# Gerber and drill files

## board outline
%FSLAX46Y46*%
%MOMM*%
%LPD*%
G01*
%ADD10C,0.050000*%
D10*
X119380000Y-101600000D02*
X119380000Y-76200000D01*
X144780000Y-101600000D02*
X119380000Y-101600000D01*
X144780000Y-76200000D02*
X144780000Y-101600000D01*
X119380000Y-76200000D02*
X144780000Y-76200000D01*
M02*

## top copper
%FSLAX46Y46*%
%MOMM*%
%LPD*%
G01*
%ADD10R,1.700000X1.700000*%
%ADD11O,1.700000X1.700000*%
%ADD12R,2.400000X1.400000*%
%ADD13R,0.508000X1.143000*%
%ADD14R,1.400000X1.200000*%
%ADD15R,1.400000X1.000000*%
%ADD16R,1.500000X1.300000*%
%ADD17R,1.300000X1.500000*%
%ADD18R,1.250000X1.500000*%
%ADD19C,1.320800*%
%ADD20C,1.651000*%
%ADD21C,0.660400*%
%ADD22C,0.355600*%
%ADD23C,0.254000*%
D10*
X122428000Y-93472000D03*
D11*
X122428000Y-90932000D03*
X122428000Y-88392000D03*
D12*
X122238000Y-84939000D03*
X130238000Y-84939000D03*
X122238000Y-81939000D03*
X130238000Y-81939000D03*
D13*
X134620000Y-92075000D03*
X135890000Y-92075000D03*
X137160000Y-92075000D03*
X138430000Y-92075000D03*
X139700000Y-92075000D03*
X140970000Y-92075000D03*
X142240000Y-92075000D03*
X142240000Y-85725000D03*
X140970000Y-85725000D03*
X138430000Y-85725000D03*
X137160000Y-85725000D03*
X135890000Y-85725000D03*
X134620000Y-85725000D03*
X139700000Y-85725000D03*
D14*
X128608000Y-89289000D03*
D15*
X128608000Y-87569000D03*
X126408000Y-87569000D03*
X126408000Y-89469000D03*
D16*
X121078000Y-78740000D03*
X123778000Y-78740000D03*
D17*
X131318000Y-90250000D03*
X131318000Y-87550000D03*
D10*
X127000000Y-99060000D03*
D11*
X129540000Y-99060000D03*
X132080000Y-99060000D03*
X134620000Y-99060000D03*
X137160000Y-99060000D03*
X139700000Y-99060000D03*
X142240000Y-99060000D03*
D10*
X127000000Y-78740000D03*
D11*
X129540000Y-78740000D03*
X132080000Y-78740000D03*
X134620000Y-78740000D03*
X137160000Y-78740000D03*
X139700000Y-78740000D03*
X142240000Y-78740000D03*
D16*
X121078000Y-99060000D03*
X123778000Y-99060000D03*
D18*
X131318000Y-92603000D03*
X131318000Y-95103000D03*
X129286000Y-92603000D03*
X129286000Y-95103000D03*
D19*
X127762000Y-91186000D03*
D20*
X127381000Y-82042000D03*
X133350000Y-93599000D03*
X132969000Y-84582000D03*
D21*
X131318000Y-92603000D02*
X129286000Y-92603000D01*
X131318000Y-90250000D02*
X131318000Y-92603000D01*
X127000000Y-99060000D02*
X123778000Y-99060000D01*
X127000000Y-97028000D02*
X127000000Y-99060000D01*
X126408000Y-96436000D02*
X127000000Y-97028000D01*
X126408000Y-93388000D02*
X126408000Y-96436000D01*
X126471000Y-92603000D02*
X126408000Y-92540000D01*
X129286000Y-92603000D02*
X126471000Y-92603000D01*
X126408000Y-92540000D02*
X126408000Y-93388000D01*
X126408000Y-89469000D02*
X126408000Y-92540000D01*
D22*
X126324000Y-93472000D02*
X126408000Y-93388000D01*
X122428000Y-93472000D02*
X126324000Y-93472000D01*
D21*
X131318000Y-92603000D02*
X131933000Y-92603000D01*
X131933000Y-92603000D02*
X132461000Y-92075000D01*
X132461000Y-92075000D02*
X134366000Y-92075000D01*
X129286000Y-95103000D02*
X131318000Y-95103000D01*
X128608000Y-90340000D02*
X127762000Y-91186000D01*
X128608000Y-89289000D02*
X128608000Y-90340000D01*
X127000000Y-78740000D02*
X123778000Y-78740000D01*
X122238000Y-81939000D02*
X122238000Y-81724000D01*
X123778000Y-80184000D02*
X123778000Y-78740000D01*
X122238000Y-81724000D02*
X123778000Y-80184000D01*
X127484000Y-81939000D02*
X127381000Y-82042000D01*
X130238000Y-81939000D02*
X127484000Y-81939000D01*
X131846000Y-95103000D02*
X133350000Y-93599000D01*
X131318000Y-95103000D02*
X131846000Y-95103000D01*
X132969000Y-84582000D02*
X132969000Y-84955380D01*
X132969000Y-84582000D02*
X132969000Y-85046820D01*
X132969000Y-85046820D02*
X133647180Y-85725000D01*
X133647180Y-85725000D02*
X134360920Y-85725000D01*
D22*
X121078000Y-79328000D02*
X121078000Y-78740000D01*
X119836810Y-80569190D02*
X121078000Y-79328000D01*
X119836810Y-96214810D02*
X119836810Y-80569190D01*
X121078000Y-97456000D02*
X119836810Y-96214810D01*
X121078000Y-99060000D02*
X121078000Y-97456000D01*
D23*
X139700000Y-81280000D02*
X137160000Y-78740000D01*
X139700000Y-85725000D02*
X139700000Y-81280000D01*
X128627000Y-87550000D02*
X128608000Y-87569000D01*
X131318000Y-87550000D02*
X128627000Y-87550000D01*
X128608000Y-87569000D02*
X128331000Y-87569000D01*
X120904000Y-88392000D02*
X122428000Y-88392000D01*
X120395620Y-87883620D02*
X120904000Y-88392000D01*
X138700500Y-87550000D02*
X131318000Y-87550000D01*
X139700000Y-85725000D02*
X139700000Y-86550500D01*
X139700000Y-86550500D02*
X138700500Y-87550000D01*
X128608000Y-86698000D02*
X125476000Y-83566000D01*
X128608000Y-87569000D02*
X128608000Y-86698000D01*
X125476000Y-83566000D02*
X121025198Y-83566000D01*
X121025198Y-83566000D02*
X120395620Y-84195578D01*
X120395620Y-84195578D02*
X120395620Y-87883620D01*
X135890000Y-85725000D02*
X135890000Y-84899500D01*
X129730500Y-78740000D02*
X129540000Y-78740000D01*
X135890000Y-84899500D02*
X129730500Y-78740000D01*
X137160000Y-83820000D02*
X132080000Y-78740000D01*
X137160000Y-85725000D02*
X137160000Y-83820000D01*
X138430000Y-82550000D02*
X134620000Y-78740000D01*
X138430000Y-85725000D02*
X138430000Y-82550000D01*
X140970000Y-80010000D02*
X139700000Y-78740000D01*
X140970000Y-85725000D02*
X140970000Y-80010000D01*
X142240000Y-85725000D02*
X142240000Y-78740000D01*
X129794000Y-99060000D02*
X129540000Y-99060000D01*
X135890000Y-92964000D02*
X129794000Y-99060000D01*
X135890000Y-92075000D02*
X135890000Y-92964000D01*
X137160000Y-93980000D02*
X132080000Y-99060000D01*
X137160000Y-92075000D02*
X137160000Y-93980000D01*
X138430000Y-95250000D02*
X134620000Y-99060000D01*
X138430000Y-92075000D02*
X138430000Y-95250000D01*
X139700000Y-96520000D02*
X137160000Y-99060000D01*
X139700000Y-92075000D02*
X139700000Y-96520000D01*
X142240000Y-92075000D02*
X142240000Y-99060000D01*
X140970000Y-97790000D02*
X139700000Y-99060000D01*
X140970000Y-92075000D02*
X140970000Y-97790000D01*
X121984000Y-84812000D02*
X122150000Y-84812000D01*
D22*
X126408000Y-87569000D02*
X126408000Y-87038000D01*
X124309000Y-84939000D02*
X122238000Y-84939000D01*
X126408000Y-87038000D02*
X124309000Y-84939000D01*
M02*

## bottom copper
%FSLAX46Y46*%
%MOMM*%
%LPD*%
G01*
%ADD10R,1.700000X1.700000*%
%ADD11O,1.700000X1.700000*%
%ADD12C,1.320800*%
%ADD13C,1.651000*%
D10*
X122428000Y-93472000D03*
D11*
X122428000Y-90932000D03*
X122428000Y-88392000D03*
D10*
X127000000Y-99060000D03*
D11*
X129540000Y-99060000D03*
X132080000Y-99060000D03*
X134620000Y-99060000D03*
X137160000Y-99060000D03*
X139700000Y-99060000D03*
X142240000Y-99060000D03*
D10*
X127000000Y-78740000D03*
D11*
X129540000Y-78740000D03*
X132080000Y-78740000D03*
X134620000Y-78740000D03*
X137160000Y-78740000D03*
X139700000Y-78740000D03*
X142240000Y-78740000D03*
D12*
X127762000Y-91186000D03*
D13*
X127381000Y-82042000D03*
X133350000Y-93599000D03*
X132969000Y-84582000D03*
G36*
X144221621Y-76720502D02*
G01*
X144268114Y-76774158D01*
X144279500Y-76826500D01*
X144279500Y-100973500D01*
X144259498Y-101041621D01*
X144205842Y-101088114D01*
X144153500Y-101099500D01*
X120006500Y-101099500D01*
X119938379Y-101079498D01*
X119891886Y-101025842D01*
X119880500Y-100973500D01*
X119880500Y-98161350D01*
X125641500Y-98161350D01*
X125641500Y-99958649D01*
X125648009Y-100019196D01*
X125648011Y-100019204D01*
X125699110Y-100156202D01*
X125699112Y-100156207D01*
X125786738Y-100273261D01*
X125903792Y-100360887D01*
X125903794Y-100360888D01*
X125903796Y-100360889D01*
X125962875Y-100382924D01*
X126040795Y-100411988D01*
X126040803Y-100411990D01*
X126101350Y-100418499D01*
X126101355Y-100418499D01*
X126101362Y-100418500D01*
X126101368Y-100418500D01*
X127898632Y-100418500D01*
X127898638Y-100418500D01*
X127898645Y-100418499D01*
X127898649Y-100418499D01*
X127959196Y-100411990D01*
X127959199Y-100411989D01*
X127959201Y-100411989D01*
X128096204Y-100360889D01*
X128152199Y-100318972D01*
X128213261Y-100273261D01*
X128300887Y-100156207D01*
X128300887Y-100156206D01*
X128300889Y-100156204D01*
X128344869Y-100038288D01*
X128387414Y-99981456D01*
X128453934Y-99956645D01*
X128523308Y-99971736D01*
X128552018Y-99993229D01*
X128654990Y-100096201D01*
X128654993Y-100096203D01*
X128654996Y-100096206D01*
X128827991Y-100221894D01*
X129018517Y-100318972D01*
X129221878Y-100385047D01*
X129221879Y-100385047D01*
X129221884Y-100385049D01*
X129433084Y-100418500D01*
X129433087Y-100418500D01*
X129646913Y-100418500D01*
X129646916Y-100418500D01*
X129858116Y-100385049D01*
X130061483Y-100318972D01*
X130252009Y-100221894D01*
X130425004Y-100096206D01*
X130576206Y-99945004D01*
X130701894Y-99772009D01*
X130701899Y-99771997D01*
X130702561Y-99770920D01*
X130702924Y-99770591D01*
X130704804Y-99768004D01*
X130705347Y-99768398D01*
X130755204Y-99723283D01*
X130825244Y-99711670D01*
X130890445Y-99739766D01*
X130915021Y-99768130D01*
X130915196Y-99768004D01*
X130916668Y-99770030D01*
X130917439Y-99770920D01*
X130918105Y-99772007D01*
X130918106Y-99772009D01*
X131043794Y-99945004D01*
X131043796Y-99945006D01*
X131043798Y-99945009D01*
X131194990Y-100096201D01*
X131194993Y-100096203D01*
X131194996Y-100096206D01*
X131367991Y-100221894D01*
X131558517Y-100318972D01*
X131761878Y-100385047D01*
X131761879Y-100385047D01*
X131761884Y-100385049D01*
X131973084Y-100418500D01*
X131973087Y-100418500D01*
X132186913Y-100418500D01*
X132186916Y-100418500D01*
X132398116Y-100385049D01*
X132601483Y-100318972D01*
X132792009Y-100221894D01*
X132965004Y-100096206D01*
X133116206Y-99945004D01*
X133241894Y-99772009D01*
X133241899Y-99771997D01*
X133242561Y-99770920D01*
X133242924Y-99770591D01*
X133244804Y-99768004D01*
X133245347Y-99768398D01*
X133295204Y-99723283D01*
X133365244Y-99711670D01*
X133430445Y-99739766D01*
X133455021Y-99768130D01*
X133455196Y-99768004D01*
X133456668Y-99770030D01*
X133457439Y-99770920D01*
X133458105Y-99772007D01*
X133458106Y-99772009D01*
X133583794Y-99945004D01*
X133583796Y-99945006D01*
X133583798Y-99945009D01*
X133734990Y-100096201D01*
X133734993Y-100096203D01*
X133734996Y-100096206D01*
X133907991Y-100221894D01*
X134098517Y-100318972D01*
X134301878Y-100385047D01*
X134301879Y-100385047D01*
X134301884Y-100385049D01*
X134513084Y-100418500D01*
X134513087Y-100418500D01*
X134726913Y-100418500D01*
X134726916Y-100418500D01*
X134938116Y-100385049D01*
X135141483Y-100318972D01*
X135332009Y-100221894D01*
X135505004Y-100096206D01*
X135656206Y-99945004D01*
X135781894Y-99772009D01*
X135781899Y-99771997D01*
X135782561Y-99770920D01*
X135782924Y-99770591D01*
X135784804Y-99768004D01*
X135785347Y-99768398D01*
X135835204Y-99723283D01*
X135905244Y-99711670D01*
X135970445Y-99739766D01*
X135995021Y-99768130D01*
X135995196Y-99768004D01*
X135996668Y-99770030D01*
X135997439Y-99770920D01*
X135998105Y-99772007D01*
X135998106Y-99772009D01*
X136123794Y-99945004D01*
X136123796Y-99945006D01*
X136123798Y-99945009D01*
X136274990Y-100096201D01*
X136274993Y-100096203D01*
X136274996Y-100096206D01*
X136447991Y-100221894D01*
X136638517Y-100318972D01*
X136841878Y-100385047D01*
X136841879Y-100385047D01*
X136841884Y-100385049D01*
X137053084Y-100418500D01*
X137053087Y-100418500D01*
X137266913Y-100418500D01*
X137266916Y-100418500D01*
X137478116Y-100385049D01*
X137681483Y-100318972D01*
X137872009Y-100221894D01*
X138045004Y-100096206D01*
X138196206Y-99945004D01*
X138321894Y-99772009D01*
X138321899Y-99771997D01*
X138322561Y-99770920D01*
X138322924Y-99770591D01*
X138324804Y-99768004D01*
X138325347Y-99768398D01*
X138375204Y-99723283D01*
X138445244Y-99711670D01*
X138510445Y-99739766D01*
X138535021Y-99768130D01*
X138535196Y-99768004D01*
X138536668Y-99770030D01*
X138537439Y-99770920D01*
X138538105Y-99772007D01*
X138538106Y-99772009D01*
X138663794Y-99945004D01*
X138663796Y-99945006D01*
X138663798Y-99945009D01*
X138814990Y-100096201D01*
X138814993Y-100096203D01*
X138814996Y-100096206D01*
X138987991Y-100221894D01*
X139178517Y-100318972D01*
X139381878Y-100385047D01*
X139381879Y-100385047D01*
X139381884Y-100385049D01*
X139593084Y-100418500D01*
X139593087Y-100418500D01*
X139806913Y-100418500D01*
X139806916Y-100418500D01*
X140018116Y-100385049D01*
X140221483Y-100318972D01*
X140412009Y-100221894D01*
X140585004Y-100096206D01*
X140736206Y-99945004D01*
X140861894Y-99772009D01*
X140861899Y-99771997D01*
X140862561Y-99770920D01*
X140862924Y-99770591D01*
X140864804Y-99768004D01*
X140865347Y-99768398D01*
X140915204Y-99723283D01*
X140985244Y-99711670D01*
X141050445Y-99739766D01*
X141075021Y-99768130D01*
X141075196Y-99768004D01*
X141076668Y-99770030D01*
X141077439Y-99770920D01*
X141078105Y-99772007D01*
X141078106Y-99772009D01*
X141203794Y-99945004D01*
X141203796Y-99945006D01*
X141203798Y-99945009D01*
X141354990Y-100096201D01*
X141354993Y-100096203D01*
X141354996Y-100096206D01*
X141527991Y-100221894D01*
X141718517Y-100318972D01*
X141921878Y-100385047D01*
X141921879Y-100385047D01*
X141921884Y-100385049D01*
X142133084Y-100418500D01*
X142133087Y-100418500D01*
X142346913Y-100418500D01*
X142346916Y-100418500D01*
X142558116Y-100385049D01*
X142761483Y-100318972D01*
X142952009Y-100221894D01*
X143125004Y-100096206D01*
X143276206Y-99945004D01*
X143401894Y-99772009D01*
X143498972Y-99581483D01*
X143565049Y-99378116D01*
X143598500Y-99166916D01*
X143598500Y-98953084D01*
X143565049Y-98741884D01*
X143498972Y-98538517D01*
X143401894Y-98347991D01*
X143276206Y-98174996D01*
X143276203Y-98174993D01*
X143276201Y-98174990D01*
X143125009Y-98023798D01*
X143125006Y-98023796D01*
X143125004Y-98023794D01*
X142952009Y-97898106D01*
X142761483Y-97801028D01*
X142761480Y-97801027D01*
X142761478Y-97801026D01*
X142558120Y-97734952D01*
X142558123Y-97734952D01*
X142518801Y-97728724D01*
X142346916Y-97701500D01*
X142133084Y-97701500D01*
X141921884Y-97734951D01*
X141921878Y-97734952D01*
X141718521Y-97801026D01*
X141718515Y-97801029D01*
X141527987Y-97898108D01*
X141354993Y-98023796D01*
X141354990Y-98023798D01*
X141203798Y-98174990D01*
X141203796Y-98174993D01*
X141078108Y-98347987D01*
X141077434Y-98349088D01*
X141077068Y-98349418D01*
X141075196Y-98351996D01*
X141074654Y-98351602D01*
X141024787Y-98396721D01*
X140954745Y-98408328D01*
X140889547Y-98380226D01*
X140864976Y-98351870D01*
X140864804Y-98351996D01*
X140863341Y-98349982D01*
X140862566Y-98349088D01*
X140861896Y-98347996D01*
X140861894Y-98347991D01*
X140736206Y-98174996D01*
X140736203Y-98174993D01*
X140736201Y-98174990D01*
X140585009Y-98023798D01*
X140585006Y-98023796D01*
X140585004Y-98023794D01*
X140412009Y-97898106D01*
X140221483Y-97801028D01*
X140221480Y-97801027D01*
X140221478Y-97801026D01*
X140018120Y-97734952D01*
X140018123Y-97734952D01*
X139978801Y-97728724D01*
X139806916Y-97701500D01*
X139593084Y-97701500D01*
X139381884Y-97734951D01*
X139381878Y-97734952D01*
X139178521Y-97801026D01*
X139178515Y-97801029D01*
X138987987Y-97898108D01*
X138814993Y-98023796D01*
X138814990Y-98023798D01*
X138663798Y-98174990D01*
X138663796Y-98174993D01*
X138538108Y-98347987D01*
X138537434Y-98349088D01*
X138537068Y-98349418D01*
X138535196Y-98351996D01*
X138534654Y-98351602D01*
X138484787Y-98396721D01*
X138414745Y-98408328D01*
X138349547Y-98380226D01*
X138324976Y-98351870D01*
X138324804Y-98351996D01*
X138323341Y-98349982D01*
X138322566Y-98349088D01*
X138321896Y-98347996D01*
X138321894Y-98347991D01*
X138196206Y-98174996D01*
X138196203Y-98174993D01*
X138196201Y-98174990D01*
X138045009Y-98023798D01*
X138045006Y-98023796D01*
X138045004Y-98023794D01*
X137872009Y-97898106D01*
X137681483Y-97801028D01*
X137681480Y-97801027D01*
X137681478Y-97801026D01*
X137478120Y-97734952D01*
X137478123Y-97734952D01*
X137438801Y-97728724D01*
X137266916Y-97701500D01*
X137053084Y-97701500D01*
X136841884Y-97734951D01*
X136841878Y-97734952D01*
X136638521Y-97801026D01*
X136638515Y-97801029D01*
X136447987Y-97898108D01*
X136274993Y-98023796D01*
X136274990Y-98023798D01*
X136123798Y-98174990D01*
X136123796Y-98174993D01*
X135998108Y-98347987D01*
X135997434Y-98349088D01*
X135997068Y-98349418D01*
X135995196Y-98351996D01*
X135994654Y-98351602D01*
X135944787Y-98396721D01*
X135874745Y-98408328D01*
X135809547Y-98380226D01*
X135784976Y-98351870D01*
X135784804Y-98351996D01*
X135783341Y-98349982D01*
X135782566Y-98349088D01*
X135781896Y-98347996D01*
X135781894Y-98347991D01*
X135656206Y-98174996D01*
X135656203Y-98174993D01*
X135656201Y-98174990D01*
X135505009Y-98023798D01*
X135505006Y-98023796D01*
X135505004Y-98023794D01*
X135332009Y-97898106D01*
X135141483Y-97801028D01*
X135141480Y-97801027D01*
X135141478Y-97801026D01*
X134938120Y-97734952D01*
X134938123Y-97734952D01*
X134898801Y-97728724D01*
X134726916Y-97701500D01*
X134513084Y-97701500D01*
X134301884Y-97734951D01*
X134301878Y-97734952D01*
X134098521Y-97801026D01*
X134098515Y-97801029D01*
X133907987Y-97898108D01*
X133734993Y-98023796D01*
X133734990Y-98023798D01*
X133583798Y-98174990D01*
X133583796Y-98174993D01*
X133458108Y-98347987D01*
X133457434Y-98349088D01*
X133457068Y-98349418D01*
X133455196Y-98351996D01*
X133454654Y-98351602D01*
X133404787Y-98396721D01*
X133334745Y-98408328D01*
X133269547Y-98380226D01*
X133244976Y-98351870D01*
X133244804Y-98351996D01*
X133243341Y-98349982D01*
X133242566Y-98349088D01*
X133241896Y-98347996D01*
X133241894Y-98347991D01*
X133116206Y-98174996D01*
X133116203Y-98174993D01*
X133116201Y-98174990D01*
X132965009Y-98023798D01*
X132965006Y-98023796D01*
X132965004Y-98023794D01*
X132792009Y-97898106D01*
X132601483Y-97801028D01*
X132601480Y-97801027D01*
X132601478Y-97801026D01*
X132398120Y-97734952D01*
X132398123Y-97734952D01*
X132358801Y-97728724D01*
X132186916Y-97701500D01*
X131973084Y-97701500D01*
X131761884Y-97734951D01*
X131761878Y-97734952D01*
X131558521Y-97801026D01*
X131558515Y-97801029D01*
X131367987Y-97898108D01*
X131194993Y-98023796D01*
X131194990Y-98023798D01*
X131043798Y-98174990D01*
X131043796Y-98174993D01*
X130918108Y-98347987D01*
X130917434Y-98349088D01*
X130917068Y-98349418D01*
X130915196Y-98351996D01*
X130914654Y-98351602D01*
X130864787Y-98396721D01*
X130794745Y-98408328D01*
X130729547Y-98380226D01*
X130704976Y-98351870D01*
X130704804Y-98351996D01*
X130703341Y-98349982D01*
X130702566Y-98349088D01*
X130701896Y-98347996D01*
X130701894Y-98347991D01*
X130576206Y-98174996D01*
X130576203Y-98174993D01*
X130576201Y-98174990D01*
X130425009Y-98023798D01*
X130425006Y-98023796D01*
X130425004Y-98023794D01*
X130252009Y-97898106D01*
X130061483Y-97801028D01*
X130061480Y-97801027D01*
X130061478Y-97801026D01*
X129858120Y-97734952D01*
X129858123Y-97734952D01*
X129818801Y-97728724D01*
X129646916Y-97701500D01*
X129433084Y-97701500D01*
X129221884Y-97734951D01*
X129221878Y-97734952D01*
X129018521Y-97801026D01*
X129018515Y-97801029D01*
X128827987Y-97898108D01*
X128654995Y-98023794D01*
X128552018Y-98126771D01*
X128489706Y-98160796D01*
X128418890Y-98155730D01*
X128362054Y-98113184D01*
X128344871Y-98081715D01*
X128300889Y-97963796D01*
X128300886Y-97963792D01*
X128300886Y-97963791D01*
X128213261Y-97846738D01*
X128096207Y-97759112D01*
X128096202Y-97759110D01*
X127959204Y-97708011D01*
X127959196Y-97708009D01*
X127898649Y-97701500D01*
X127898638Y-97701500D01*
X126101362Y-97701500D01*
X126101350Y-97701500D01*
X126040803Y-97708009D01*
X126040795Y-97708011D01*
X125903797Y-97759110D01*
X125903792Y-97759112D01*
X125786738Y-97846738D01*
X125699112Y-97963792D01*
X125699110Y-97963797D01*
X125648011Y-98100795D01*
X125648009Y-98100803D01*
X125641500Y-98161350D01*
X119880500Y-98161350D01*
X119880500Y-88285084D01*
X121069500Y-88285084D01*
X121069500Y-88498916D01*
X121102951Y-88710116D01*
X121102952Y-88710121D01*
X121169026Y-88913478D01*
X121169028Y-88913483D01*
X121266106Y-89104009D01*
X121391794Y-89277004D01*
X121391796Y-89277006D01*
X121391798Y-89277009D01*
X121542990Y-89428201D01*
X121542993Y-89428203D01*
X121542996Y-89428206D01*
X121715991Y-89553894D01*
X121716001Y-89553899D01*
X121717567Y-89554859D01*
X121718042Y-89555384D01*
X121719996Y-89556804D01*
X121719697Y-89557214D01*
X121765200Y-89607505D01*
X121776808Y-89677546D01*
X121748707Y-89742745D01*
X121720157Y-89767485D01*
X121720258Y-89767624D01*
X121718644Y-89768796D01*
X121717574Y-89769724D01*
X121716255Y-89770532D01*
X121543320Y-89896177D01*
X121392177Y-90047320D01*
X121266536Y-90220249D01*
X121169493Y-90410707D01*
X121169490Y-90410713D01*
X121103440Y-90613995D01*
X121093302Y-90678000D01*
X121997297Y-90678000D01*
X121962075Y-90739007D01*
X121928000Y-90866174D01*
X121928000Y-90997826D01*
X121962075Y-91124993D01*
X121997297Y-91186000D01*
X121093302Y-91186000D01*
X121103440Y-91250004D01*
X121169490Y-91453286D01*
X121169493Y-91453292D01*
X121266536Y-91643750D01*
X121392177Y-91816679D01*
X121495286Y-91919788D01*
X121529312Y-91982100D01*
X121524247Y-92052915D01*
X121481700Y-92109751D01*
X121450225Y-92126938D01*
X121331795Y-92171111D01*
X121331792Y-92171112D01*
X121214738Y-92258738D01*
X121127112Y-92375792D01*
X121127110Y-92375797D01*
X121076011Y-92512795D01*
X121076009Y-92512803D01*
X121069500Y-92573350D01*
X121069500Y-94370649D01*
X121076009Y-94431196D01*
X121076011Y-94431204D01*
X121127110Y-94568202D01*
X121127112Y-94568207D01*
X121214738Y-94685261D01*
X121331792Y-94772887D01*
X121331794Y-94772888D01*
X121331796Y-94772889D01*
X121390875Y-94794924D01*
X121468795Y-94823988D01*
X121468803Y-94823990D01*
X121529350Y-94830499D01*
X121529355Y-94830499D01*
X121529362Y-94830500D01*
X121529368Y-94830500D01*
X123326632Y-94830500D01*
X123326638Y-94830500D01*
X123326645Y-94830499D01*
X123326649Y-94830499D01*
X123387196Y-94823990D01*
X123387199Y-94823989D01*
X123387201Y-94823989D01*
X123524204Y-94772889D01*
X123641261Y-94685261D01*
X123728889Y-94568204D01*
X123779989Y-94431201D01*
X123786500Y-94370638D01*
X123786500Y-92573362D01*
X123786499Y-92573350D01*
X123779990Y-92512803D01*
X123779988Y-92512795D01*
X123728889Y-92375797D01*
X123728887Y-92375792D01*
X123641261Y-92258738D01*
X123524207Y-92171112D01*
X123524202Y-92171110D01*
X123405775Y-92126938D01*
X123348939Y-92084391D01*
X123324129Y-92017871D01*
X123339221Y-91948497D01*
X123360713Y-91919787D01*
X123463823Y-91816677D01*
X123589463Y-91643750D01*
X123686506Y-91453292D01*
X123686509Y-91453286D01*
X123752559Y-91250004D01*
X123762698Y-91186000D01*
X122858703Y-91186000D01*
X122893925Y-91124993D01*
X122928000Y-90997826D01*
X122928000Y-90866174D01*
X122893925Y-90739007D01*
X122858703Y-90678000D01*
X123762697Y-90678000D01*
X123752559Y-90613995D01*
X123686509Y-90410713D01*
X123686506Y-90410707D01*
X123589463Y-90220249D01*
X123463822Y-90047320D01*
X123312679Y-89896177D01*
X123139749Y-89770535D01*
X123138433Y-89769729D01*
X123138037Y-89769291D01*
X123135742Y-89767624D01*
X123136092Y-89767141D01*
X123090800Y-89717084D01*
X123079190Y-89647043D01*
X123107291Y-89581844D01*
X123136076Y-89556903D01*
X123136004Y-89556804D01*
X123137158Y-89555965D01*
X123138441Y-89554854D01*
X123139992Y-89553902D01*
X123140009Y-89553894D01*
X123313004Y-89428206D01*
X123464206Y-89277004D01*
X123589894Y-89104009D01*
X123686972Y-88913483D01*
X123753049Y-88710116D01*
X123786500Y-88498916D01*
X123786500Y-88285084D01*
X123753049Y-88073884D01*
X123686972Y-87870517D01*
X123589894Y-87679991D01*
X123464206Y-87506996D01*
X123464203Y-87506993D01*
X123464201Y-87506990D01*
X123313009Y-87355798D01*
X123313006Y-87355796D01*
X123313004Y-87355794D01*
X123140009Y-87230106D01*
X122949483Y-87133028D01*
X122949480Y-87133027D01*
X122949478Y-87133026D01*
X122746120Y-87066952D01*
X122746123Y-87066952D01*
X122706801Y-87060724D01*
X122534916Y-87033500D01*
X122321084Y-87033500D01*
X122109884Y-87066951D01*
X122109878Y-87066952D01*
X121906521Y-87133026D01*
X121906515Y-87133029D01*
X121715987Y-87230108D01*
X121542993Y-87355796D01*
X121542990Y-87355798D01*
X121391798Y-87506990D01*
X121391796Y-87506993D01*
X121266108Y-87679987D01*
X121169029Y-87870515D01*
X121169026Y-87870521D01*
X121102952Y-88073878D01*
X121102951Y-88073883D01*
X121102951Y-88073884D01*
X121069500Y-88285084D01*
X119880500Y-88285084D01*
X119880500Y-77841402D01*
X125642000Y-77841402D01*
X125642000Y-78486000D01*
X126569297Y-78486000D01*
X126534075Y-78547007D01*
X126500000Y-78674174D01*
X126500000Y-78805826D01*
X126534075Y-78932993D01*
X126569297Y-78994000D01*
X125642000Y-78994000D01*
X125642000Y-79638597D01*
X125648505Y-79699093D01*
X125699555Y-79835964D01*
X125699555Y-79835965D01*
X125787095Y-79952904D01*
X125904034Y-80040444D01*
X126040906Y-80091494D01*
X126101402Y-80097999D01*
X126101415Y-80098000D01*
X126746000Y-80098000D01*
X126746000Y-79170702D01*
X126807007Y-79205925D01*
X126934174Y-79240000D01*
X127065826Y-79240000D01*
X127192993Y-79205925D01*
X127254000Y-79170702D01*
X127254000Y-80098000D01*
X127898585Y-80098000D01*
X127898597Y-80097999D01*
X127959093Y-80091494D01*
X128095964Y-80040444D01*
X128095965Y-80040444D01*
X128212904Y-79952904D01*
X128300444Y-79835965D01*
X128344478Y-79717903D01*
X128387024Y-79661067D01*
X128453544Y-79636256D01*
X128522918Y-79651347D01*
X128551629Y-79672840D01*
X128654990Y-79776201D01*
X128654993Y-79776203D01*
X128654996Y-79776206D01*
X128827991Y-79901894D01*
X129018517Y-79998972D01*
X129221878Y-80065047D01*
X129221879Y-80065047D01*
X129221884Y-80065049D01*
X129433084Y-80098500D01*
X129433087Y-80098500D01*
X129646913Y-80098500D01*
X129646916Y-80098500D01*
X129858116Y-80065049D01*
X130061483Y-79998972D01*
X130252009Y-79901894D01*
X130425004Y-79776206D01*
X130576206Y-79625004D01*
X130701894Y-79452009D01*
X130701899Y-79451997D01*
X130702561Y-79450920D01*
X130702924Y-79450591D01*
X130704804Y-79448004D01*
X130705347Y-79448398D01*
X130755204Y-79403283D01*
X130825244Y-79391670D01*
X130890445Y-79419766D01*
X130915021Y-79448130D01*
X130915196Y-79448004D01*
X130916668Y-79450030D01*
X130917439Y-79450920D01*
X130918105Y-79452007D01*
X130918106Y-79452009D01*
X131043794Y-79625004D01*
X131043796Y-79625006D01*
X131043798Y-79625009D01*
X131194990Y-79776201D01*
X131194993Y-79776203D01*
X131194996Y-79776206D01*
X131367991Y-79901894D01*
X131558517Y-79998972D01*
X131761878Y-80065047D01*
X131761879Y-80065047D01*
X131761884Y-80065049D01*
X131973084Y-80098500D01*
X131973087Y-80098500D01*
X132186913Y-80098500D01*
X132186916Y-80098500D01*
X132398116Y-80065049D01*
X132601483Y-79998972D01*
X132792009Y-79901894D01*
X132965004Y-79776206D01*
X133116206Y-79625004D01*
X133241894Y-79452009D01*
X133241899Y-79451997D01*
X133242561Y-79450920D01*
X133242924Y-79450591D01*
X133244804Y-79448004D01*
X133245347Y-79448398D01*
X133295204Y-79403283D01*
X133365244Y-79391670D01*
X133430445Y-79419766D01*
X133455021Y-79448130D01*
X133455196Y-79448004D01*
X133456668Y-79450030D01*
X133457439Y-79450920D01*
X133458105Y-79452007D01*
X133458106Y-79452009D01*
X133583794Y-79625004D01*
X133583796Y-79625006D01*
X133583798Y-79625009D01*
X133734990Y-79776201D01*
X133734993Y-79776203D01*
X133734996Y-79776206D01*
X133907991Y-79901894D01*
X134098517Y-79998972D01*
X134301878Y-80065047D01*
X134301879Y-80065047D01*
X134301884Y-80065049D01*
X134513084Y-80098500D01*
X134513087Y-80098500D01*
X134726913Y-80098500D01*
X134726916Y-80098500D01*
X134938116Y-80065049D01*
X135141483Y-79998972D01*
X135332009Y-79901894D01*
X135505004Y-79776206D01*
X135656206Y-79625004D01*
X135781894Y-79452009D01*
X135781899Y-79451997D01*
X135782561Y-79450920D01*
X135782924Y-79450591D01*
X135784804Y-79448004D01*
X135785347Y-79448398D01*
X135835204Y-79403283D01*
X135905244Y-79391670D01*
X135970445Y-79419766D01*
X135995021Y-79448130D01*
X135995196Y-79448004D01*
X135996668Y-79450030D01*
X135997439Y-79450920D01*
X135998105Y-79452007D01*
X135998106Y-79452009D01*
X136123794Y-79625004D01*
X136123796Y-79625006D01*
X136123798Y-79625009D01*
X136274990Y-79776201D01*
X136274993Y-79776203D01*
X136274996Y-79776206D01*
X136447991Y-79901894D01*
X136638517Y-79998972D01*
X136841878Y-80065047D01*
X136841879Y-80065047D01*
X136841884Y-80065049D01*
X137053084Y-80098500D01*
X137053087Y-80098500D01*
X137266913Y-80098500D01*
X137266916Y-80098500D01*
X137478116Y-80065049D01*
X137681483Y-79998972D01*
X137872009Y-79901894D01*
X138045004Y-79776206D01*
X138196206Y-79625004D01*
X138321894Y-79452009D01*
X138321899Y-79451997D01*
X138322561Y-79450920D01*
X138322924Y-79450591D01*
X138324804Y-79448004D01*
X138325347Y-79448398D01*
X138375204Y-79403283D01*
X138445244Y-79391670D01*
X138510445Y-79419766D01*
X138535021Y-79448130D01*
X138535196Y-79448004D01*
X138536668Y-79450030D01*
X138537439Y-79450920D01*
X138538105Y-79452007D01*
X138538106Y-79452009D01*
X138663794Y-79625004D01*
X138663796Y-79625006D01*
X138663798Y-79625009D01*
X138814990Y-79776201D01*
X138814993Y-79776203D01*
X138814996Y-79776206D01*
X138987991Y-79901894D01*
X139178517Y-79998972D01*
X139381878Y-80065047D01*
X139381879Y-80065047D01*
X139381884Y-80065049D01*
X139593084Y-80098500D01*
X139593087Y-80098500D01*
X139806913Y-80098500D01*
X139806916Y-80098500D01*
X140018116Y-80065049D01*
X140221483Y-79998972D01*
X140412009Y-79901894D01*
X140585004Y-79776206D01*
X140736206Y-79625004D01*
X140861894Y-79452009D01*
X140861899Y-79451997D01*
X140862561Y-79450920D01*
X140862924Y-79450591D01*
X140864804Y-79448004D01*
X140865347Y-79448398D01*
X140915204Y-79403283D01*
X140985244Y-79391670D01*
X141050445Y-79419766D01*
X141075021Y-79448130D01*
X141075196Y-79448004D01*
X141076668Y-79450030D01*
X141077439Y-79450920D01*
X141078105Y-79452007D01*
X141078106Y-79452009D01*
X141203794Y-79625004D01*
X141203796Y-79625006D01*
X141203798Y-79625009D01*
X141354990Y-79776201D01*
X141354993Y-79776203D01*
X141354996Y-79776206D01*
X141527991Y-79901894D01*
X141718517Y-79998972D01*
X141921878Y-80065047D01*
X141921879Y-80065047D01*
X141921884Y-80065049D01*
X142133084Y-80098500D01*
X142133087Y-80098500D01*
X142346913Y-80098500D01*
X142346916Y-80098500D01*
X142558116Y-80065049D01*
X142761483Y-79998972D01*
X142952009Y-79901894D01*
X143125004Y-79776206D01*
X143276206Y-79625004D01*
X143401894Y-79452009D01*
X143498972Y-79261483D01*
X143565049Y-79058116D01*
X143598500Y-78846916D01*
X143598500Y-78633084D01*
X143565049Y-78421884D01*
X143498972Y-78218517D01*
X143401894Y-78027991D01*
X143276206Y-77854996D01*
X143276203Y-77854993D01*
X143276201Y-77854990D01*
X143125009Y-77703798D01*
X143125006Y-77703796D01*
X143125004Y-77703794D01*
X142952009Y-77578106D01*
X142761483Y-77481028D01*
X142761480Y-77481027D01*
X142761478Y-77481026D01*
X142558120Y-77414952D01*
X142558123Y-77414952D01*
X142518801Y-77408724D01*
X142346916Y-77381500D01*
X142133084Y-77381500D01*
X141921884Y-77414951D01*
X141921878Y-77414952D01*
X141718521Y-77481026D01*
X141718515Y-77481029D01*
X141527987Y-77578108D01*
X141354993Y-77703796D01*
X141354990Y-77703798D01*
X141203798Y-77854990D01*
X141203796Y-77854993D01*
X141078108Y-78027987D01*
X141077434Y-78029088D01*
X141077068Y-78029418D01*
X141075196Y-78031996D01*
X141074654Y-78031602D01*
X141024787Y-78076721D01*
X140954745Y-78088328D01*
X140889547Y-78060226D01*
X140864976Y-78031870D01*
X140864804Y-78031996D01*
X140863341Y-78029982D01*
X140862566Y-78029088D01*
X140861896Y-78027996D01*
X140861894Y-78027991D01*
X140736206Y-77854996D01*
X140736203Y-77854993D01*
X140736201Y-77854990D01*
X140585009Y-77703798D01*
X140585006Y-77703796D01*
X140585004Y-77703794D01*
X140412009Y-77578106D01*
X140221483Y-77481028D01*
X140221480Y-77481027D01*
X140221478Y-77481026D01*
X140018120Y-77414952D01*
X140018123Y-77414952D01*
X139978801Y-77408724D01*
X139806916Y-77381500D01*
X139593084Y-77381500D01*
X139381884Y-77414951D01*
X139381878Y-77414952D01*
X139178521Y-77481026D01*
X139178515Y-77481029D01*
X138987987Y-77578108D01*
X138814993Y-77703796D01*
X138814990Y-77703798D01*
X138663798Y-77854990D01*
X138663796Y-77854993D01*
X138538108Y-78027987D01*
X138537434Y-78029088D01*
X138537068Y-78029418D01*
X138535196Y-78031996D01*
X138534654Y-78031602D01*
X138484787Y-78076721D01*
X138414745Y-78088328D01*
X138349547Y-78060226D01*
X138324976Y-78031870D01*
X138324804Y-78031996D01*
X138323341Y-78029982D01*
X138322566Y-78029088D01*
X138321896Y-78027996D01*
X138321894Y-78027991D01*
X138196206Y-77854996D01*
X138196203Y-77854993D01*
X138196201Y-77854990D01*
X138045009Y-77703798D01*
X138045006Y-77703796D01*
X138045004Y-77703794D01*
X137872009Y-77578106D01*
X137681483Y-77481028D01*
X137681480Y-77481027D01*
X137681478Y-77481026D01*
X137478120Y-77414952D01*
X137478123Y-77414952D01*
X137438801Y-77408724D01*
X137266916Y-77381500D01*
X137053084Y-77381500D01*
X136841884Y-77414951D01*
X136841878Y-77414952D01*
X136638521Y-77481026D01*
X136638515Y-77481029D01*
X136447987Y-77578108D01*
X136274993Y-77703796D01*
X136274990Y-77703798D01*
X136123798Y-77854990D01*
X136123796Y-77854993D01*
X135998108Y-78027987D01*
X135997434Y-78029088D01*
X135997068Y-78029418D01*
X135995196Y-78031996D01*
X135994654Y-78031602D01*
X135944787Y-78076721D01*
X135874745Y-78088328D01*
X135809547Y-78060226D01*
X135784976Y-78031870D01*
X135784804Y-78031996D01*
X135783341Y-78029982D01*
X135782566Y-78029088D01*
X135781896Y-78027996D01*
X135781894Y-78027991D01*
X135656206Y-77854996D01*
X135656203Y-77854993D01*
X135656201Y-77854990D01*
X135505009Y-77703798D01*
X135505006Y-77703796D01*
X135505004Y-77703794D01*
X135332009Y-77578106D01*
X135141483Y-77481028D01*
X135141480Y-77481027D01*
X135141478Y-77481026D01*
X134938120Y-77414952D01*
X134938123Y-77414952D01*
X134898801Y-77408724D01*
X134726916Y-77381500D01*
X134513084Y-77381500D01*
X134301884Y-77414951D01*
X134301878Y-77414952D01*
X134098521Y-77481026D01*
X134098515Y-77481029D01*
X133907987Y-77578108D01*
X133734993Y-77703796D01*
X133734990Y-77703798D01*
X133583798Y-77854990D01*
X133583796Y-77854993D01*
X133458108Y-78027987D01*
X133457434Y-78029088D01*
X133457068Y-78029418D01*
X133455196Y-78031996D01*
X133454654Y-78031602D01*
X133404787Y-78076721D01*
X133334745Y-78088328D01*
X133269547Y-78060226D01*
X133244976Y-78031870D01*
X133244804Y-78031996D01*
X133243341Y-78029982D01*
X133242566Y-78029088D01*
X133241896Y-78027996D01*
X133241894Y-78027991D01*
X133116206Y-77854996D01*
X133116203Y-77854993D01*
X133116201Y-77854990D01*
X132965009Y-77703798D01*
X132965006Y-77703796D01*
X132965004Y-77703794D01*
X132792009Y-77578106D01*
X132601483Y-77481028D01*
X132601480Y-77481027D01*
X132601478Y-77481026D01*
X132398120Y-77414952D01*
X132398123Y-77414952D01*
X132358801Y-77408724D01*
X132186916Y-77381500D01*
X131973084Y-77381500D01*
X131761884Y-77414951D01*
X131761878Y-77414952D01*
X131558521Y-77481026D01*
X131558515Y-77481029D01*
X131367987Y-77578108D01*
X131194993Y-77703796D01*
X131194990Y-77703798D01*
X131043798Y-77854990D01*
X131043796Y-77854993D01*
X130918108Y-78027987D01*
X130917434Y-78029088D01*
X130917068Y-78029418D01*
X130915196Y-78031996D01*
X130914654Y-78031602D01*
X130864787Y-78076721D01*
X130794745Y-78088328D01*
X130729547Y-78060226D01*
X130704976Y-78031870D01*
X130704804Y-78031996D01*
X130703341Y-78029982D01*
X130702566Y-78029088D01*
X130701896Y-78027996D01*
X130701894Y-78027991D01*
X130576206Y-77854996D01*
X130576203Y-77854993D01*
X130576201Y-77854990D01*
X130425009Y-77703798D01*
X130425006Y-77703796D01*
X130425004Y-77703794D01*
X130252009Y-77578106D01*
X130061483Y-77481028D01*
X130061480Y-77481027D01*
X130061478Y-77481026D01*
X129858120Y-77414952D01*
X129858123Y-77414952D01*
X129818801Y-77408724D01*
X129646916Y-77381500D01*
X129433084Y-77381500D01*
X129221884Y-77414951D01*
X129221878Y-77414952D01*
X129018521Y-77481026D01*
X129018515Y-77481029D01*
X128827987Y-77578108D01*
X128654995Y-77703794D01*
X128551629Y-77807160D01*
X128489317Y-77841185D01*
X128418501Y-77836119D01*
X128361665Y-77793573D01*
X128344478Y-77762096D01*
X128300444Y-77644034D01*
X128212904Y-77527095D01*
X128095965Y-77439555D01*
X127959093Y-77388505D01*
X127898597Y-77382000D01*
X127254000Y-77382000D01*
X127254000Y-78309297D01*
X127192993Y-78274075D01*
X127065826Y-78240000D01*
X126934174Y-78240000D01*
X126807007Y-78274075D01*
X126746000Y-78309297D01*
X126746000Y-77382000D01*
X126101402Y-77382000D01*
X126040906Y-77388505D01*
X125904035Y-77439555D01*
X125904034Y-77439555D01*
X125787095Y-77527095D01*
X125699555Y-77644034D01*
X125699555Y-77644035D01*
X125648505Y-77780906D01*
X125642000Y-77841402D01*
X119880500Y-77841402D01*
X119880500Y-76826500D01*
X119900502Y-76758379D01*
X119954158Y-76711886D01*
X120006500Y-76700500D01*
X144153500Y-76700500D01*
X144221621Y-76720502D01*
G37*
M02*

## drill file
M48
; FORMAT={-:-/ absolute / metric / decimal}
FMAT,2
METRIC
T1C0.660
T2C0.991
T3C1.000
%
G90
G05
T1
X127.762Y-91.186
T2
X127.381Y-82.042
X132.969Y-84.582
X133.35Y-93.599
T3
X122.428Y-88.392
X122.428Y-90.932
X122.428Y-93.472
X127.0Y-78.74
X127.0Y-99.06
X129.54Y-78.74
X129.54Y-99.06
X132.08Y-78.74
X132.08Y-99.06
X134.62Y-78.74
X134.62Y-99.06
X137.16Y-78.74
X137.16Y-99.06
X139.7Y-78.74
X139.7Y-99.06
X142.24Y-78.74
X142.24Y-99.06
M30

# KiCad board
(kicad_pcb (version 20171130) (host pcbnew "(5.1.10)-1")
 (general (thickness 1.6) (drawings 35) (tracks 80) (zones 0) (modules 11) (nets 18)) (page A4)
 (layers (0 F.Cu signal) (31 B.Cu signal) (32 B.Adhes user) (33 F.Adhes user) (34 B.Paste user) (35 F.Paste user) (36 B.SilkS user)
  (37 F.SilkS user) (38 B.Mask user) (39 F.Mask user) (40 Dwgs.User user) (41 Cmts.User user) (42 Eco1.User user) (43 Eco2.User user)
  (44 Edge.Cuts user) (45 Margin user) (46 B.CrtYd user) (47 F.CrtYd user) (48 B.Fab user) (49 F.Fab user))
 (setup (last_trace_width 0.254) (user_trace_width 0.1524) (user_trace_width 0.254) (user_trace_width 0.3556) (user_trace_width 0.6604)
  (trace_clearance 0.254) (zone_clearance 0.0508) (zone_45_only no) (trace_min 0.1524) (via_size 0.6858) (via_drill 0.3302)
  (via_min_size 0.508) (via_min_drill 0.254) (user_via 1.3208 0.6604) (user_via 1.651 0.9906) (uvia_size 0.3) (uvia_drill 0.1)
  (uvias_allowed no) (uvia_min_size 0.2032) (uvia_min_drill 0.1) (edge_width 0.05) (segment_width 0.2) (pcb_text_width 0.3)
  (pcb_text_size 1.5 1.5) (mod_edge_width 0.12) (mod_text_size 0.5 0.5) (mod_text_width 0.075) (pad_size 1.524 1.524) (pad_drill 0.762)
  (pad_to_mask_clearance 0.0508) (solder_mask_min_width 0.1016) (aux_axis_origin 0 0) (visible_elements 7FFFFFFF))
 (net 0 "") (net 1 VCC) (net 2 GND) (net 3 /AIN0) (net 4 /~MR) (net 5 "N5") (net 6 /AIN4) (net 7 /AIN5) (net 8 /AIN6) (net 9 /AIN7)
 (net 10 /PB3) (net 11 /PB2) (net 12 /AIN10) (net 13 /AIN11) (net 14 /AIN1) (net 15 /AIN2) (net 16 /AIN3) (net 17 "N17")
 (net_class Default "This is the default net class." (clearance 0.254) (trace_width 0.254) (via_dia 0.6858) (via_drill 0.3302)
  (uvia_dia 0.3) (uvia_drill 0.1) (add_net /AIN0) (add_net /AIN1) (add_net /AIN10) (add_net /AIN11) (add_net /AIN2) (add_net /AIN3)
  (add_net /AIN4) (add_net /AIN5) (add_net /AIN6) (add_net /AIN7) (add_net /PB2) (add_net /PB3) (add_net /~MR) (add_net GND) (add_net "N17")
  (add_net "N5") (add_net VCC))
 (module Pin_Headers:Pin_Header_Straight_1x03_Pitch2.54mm (layer F.Cu) (at 122.428 93.472 180)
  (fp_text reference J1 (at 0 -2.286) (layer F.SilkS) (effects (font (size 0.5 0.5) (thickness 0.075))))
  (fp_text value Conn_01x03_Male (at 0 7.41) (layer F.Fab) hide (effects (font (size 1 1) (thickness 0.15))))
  (pad 1 thru_hole rect (at 0 0 180) (size 1.7 1.7) (drill 1) (layers *.Cu *.Mask) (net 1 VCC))
  (pad 2 thru_hole oval (at 0 2.54 180) (size 1.7 1.7) (drill 1) (layers *.Cu *.Mask) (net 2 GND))
  (pad 3 thru_hole oval (at 0 5.08 180) (size 1.7 1.7) (drill 1) (layers *.Cu *.Mask) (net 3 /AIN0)))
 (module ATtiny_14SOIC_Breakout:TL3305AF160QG (layer F.Cu) (at 126.238 83.439)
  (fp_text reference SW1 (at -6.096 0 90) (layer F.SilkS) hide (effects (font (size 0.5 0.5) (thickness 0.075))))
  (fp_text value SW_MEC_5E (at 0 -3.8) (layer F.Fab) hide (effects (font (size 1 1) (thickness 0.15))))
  (pad 1 smd rect (at -4 1.5) (size 2.4 1.4) (layers F.Cu F.Paste F.Mask) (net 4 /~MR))
  (pad 2 smd rect (at 4 1.5) (size 2.4 1.4) (layers F.Cu F.Paste F.Mask) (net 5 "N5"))
  (pad 3 smd rect (at -4 -1.5) (size 2.4 1.4) (layers F.Cu F.Paste F.Mask) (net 2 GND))
  (pad 4 smd rect (at 4 -1.5) (size 2.4 1.4) (layers F.Cu F.Paste F.Mask) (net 2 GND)))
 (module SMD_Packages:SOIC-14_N (layer F.Cu) (at 138.43 88.773)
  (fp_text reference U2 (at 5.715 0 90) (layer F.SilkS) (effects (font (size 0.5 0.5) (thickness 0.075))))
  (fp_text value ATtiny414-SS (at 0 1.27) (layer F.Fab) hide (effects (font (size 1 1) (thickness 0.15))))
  (pad 1 smd rect (at -3.81 3.302) (size 0.508 1.143) (layers F.Cu F.Paste F.Mask) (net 1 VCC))
  (pad 2 smd rect (at -2.54 3.302) (size 0.508 1.143) (layers F.Cu F.Paste F.Mask) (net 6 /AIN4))
  (pad 3 smd rect (at -1.27 3.302) (size 0.508 1.143) (layers F.Cu F.Paste F.Mask) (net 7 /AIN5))
  (pad 4 smd rect (at 0 3.302) (size 0.508 1.143) (layers F.Cu F.Paste F.Mask) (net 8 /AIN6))
  (pad 5 smd rect (at 1.27 3.302) (size 0.508 1.143) (layers F.Cu F.Paste F.Mask) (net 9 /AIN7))
  (pad 6 smd rect (at 2.54 3.302) (size 0.508 1.143) (layers F.Cu F.Paste F.Mask) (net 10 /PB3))
  (pad 7 smd rect (at 3.81 3.302) (size 0.508 1.143) (layers F.Cu F.Paste F.Mask) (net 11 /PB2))
  (pad 8 smd rect (at 3.81 -3.048) (size 0.508 1.143) (layers F.Cu F.Paste F.Mask) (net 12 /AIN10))
  (pad 9 smd rect (at 2.54 -3.048) (size 0.508 1.143) (layers F.Cu F.Paste F.Mask) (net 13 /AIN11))
  (pad 11 smd rect (at 0 -3.048) (size 0.508 1.143) (layers F.Cu F.Paste F.Mask) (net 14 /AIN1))
  (pad 12 smd rect (at -1.27 -3.048) (size 0.508 1.143) (layers F.Cu F.Paste F.Mask) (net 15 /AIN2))
  (pad 13 smd rect (at -2.54 -3.048) (size 0.508 1.143) (layers F.Cu F.Paste F.Mask) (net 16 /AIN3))
  (pad 14 smd rect (at -3.81 -3.048) (size 0.508 1.143) (layers F.Cu F.Paste F.Mask) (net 2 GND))
  (pad 10 smd rect (at 1.27 -3.048) (size 0.508 1.143) (layers F.Cu F.Paste F.Mask) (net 3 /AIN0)))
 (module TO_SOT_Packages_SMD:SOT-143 (layer F.Cu) (at 127.508 88.519 180)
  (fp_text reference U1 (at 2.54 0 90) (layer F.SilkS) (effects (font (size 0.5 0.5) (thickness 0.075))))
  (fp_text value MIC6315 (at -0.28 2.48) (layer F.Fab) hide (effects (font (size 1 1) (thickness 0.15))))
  (pad 1 smd rect (at -1.1 -0.77 90) (size 1.2 1.4) (layers F.Cu F.Paste F.Mask) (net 2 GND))
  (pad 2 smd rect (at -1.1 0.95 90) (size 1 1.4) (layers F.Cu F.Paste F.Mask) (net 3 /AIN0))
  (pad 3 smd rect (at 1.1 0.95 90) (size 1 1.4) (layers F.Cu F.Paste F.Mask) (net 4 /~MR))
  (pad 4 smd rect (at 1.1 -0.95 90) (size 1 1.4) (layers F.Cu F.Paste F.Mask) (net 1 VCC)))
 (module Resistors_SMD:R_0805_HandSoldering (layer F.Cu) (at 122.428 78.74)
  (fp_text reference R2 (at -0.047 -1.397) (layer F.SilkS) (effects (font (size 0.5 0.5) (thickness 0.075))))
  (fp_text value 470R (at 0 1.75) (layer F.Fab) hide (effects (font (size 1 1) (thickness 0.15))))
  (pad 1 smd rect (at -1.35 0) (size 1.5 1.3) (layers F.Cu F.Paste F.Mask) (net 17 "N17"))
  (pad 2 smd rect (at 1.35 0) (size 1.5 1.3) (layers F.Cu F.Paste F.Mask) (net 2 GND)))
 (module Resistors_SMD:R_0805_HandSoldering (layer F.Cu) (at 131.318 88.9 90)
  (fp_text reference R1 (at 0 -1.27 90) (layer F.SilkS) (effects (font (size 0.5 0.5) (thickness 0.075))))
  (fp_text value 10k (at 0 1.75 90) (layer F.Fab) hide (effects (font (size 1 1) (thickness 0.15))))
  (pad 1 smd rect (at -1.35 0 90) (size 1.5 1.3) (layers F.Cu F.Paste F.Mask) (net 1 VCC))
  (pad 2 smd rect (at 1.35 0 90) (size 1.5 1.3) (layers F.Cu F.Paste F.Mask) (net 3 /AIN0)))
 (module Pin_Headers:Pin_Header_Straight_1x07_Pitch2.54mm (layer B.Cu) (at 127 99.06 270)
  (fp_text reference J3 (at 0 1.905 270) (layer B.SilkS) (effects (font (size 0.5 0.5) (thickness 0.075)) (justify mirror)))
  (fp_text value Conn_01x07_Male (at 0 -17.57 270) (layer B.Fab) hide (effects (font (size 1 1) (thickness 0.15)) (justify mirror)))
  (pad 1 thru_hole rect (at 0 0 270) (size 1.7 1.7) (drill 1) (layers *.Cu *.Mask) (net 1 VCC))
  (pad 2 thru_hole oval (at 0 -2.54 270) (size 1.7 1.7) (drill 1) (layers *.Cu *.Mask) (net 6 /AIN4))
  (pad 3 thru_hole oval (at 0 -5.08 270) (size 1.7 1.7) (drill 1) (layers *.Cu *.Mask) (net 7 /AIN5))
  (pad 4 thru_hole oval (at 0 -7.62 270) (size 1.7 1.7) (drill 1) (layers *.Cu *.Mask) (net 8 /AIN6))
  (pad 5 thru_hole oval (at 0 -10.16 270) (size 1.7 1.7) (drill 1) (layers *.Cu *.Mask) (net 9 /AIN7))
  (pad 6 thru_hole oval (at 0 -12.7 270) (size 1.7 1.7) (drill 1) (layers *.Cu *.Mask) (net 10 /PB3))
  (pad 7 thru_hole oval (at 0 -15.24 270) (size 1.7 1.7) (drill 1) (layers *.Cu *.Mask) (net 11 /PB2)))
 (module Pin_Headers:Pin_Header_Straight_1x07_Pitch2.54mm (layer B.Cu) (at 127 78.74 270)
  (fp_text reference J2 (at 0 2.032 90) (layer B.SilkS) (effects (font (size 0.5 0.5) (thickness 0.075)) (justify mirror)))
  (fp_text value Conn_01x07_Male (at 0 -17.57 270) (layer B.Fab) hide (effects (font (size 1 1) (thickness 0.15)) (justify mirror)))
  (pad 1 thru_hole rect (at 0 0 270) (size 1.7 1.7) (drill 1) (layers *.Cu *.Mask) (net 2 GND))
  (pad 2 thru_hole oval (at 0 -2.54 270) (size 1.7 1.7) (drill 1) (layers *.Cu *.Mask) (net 16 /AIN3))
  (pad 3 thru_hole oval (at 0 -5.08 270) (size 1.7 1.7) (drill 1) (layers *.Cu *.Mask) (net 15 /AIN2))
  (pad 4 thru_hole oval (at 0 -7.62 270) (size 1.7 1.7) (drill 1) (layers *.Cu *.Mask) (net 14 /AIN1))
  (pad 5 thru_hole oval (at 0 -10.16 270) (size 1.7 1.7) (drill 1) (layers *.Cu *.Mask) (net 3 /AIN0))
  (pad 6 thru_hole oval (at 0 -12.7 270) (size 1.7 1.7) (drill 1) (layers *.Cu *.Mask) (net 13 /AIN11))
  (pad 7 thru_hole oval (at 0 -15.24 270) (size 1.7 1.7) (drill 1) (layers *.Cu *.Mask) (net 12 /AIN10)))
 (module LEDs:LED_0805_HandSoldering (layer F.Cu) (at 122.428 99.06)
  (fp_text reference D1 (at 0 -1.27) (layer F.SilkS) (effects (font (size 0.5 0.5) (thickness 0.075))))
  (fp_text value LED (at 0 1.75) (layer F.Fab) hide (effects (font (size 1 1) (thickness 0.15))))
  (pad 1 smd rect (at -1.35 0) (size 1.5 1.3) (layers F.Cu F.Paste F.Mask) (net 17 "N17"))
  (pad 2 smd rect (at 1.35 0) (size 1.5 1.3) (layers F.Cu F.Paste F.Mask) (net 1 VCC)))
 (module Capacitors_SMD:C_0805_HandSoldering (layer F.Cu) (at 131.318 93.853 270)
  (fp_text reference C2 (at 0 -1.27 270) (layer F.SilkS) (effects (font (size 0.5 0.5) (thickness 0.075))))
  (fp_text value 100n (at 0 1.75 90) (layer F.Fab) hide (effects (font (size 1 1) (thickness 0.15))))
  (pad 1 smd rect (at -1.25 0 270) (size 1.5 1.25) (layers F.Cu F.Paste F.Mask) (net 1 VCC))
  (pad 2 smd rect (at 1.25 0 270) (size 1.5 1.25) (layers F.Cu F.Paste F.Mask) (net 2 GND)))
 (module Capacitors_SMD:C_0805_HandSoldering (layer F.Cu) (at 129.286 93.853 270)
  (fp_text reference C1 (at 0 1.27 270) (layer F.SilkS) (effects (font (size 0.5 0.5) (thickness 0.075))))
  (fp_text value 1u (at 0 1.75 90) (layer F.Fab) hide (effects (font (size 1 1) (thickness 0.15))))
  (pad 1 smd rect (at -1.25 0 270) (size 1.5 1.25) (layers F.Cu F.Paste F.Mask) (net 1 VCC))
  (pad 2 smd rect (at 1.25 0 270) (size 1.5 1.25) (layers F.Cu F.Paste F.Mask) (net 2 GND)))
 (gr_line (start 119.38 101.6) (end 119.38 76.2) (layer Edge.Cuts) (width 0.05))
 (gr_line (start 144.78 101.6) (end 119.38 101.6) (layer Edge.Cuts) (width 0.05))
 (gr_line (start 144.78 76.2) (end 144.78 101.6) (layer Edge.Cuts) (width 0.05))
 (gr_line (start 119.38 76.2) (end 144.78 76.2) (layer Edge.Cuts) (width 0.05))
 (segment (start 131.318 92.603) (end 129.286 92.603) (width 0.6604) (layer F.Cu) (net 1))
 (segment (start 131.318 90.25) (end 131.318 92.603) (width 0.6604) (layer F.Cu) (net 1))
 (segment (start 127 99.06) (end 123.778 99.06) (width 0.6604) (layer F.Cu) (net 1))
 (segment (start 127 97.028) (end 127 99.06) (width 0.6604) (layer F.Cu) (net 1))
 (segment (start 126.408 96.436) (end 127 97.028) (width 0.6604) (layer F.Cu) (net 1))
 (segment (start 126.408 93.388) (end 126.408 96.436) (width 0.6604) (layer F.Cu) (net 1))
 (segment (start 126.471 92.603) (end 126.408 92.54) (width 0.6604) (layer F.Cu) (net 1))
 (segment (start 129.286 92.603) (end 126.471 92.603) (width 0.6604) (layer F.Cu) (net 1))
 (segment (start 126.408 92.54) (end 126.408 93.388) (width 0.6604) (layer F.Cu) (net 1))
 (segment (start 126.408 89.469) (end 126.408 92.54) (width 0.6604) (layer F.Cu) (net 1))
 (segment (start 126.324 93.472) (end 126.408 93.388) (width 0.3556) (layer F.Cu) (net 1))
 (segment (start 122.428 93.472) (end 126.324 93.472) (width 0.3556) (layer F.Cu) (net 1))
 (segment (start 131.318 92.603) (end 131.933 92.603) (width 0.6604) (layer F.Cu) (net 1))
 (segment (start 131.933 92.603) (end 132.461 92.075) (width 0.6604) (layer F.Cu) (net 1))
 (segment (start 132.461 92.075) (end 134.366 92.075) (width 0.6604) (layer F.Cu) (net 1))
 (segment (start 129.286 95.103) (end 131.318 95.103) (width 0.6604) (layer F.Cu) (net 2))
 (via (at 127.762 91.186) (size 1.3208) (drill 0.6604) (layers F.Cu B.Cu) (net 2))
 (segment (start 128.608 90.34) (end 127.762 91.186) (width 0.6604) (layer F.Cu) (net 2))
 (segment (start 128.608 89.289) (end 128.608 90.34) (width 0.6604) (layer F.Cu) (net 2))
 (segment (start 127 78.74) (end 123.778 78.74) (width 0.6604) (layer F.Cu) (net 2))
 (segment (start 122.238 81.939) (end 122.238 81.724) (width 0.6604) (layer F.Cu) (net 2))
 (segment (start 123.778 80.184) (end 123.778 78.74) (width 0.6604) (layer F.Cu) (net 2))
 (segment (start 122.238 81.724) (end 123.778 80.184) (width 0.6604) (layer F.Cu) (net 2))
 (via (at 127.381 82.042) (size 1.651) (drill 0.9906) (layers F.Cu B.Cu) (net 2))
 (segment (start 127.484 81.939) (end 127.381 82.042) (width 0.6604) (layer F.Cu) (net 2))
 (segment (start 130.238 81.939) (end 127.484 81.939) (width 0.6604) (layer F.Cu) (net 2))
 (via (at 133.35 93.599) (size 1.651) (drill 0.9906) (layers F.Cu B.Cu) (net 2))
 (segment (start 131.846 95.103) (end 133.35 93.599) (width 0.6604) (layer F.Cu) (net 2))
 (segment (start 131.318 95.103) (end 131.846 95.103) (width 0.6604) (layer F.Cu) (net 2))
 (via (at 132.969 84.582) (size 1.651) (drill 0.9906) (layers F.Cu B.Cu) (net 2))
 (segment (start 132.969 84.582) (end 132.969 84.95538) (width 0.6604) (layer F.Cu) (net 2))
 (segment (start 132.969 84.582) (end 132.969 85.04682) (width 0.6604) (layer F.Cu) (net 2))
 (segment (start 132.969 85.04682) (end 133.64718 85.725) (width 0.6604) (layer F.Cu) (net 2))
 (segment (start 133.64718 85.725) (end 134.36092 85.725) (width 0.6604) (layer F.Cu) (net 2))
 (segment (start 121.078 79.328) (end 121.078 78.74) (width 0.3556) (layer F.Cu) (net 17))
 (segment (start 119.83681 80.56919) (end 121.078 79.328) (width 0.3556) (layer F.Cu) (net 17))
 (segment (start 119.83681 96.21481) (end 119.83681 80.56919) (width 0.3556) (layer F.Cu) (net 17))
 (segment (start 121.078 97.456) (end 119.83681 96.21481) (width 0.3556) (layer F.Cu) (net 17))
 (segment (start 121.078 99.06) (end 121.078 97.456) (width 0.3556) (layer F.Cu) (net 17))
 (segment (start 139.7 81.28) (end 137.16 78.74) (width 0.254) (layer F.Cu) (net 3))
 (segment (start 139.7 85.725) (end 139.7 81.28) (width 0.254) (layer F.Cu) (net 3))
 (segment (start 128.627 87.55) (end 128.608 87.569) (width 0.254) (layer F.Cu) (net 3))
 (segment (start 131.318 87.55) (end 128.627 87.55) (width 0.254) (layer F.Cu) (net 3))
 (segment (start 128.608 87.569) (end 128.331 87.569) (width 0.254) (layer F.Cu) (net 3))
 (segment (start 120.904 88.392) (end 122.428 88.392) (width 0.254) (layer F.Cu) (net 3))
 (segment (start 120.39562 87.88362) (end 120.904 88.392) (width 0.254) (layer F.Cu) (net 3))
 (segment (start 138.7005 87.55) (end 131.318 87.55) (width 0.254) (layer F.Cu) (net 3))
 (segment (start 139.7 85.725) (end 139.7 86.5505) (width 0.254) (layer F.Cu) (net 3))
 (segment (start 139.7 86.5505) (end 138.7005 87.55) (width 0.254) (layer F.Cu) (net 3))
 (segment (start 128.608 86.698) (end 125.476 83.566) (width 0.254) (layer F.Cu) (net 3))
 (segment (start 128.608 87.569) (end 128.608 86.698) (width 0.254) (layer F.Cu) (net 3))
 (segment (start 125.476 83.566) (end 121.025198 83.566) (width 0.254) (layer F.Cu) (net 3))
 (segment (start 121.025198 83.566) (end 120.39562 84.195578) (width 0.254) (layer F.Cu) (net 3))
 (segment (start 120.39562 84.195578) (end 120.39562 87.88362) (width 0.254) (layer F.Cu) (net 3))
 (segment (start 135.89 85.725) (end 135.89 84.8995) (width 0.254) (layer F.Cu) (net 16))
 (segment (start 129.7305 78.74) (end 129.54 78.74) (width 0.254) (layer F.Cu) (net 16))
 (segment (start 135.89 84.8995) (end 129.7305 78.74) (width 0.254) (layer F.Cu) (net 16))
 (segment (start 137.16 83.82) (end 132.08 78.74) (width 0.254) (layer F.Cu) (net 15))
 (segment (start 137.16 85.725) (end 137.16 83.82) (width 0.254) (layer F.Cu) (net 15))
 (segment (start 138.43 82.55) (end 134.62 78.74) (width 0.254) (layer F.Cu) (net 14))
 (segment (start 138.43 85.725) (end 138.43 82.55) (width 0.254) (layer F.Cu) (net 14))
 (segment (start 140.97 80.01) (end 139.7 78.74) (width 0.254) (layer F.Cu) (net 13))
 (segment (start 140.97 85.725) (end 140.97 80.01) (width 0.254) (layer F.Cu) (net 13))
 (segment (start 142.24 85.725) (end 142.24 78.74) (width 0.254) (layer F.Cu) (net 12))
 (segment (start 129.794 99.06) (end 129.54 99.06) (width 0.254) (layer F.Cu) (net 6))
 (segment (start 135.89 92.964) (end 129.794 99.06) (width 0.254) (layer F.Cu) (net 6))
 (segment (start 135.89 92.075) (end 135.89 92.964) (width 0.254) (layer F.Cu) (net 6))
 (segment (start 137.16 93.98) (end 132.08 99.06) (width 0.254) (layer F.Cu) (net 7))
 (segment (start 137.16 92.075) (end 137.16 93.98) (width 0.254) (layer F.Cu) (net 7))
 (segment (start 138.43 95.25) (end 134.62 99.06) (width 0.254) (layer F.Cu) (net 8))
 (segment (start 138.43 92.075) (end 138.43 95.25) (width 0.254) (layer F.Cu) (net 8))
 (segment (start 139.7 96.52) (end 137.16 99.06) (width 0.254) (layer F.Cu) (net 9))
 (segment (start 139.7 92.075) (end 139.7 96.52) (width 0.254) (layer F.Cu) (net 9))
 (segment (start 142.24 92.075) (end 142.24 99.06) (width 0.254) (layer F.Cu) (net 11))
 (segment (start 140.97 97.79) (end 139.7 99.06) (width 0.254) (layer F.Cu) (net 10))
 (segment (start 140.97 92.075) (end 140.97 97.79) (width 0.254) (layer F.Cu) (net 10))
 (segment (start 121.984 84.812) (end 122.15 84.812) (width 0.254) (layer F.Cu) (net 4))
 (segment (start 126.408 87.569) (end 126.408 87.038) (width 0.3556) (layer F.Cu) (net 4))
 (segment (start 124.309 84.939) (end 122.238 84.939) (width 0.3556) (layer F.Cu) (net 4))
 (segment (start 126.408 87.038) (end 124.309 84.939) (width 0.3556) (layer F.Cu) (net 4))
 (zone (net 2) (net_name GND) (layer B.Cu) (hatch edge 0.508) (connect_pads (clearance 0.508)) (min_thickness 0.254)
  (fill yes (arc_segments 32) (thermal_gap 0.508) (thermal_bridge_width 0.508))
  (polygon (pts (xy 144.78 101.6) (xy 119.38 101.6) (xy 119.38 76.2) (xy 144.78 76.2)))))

